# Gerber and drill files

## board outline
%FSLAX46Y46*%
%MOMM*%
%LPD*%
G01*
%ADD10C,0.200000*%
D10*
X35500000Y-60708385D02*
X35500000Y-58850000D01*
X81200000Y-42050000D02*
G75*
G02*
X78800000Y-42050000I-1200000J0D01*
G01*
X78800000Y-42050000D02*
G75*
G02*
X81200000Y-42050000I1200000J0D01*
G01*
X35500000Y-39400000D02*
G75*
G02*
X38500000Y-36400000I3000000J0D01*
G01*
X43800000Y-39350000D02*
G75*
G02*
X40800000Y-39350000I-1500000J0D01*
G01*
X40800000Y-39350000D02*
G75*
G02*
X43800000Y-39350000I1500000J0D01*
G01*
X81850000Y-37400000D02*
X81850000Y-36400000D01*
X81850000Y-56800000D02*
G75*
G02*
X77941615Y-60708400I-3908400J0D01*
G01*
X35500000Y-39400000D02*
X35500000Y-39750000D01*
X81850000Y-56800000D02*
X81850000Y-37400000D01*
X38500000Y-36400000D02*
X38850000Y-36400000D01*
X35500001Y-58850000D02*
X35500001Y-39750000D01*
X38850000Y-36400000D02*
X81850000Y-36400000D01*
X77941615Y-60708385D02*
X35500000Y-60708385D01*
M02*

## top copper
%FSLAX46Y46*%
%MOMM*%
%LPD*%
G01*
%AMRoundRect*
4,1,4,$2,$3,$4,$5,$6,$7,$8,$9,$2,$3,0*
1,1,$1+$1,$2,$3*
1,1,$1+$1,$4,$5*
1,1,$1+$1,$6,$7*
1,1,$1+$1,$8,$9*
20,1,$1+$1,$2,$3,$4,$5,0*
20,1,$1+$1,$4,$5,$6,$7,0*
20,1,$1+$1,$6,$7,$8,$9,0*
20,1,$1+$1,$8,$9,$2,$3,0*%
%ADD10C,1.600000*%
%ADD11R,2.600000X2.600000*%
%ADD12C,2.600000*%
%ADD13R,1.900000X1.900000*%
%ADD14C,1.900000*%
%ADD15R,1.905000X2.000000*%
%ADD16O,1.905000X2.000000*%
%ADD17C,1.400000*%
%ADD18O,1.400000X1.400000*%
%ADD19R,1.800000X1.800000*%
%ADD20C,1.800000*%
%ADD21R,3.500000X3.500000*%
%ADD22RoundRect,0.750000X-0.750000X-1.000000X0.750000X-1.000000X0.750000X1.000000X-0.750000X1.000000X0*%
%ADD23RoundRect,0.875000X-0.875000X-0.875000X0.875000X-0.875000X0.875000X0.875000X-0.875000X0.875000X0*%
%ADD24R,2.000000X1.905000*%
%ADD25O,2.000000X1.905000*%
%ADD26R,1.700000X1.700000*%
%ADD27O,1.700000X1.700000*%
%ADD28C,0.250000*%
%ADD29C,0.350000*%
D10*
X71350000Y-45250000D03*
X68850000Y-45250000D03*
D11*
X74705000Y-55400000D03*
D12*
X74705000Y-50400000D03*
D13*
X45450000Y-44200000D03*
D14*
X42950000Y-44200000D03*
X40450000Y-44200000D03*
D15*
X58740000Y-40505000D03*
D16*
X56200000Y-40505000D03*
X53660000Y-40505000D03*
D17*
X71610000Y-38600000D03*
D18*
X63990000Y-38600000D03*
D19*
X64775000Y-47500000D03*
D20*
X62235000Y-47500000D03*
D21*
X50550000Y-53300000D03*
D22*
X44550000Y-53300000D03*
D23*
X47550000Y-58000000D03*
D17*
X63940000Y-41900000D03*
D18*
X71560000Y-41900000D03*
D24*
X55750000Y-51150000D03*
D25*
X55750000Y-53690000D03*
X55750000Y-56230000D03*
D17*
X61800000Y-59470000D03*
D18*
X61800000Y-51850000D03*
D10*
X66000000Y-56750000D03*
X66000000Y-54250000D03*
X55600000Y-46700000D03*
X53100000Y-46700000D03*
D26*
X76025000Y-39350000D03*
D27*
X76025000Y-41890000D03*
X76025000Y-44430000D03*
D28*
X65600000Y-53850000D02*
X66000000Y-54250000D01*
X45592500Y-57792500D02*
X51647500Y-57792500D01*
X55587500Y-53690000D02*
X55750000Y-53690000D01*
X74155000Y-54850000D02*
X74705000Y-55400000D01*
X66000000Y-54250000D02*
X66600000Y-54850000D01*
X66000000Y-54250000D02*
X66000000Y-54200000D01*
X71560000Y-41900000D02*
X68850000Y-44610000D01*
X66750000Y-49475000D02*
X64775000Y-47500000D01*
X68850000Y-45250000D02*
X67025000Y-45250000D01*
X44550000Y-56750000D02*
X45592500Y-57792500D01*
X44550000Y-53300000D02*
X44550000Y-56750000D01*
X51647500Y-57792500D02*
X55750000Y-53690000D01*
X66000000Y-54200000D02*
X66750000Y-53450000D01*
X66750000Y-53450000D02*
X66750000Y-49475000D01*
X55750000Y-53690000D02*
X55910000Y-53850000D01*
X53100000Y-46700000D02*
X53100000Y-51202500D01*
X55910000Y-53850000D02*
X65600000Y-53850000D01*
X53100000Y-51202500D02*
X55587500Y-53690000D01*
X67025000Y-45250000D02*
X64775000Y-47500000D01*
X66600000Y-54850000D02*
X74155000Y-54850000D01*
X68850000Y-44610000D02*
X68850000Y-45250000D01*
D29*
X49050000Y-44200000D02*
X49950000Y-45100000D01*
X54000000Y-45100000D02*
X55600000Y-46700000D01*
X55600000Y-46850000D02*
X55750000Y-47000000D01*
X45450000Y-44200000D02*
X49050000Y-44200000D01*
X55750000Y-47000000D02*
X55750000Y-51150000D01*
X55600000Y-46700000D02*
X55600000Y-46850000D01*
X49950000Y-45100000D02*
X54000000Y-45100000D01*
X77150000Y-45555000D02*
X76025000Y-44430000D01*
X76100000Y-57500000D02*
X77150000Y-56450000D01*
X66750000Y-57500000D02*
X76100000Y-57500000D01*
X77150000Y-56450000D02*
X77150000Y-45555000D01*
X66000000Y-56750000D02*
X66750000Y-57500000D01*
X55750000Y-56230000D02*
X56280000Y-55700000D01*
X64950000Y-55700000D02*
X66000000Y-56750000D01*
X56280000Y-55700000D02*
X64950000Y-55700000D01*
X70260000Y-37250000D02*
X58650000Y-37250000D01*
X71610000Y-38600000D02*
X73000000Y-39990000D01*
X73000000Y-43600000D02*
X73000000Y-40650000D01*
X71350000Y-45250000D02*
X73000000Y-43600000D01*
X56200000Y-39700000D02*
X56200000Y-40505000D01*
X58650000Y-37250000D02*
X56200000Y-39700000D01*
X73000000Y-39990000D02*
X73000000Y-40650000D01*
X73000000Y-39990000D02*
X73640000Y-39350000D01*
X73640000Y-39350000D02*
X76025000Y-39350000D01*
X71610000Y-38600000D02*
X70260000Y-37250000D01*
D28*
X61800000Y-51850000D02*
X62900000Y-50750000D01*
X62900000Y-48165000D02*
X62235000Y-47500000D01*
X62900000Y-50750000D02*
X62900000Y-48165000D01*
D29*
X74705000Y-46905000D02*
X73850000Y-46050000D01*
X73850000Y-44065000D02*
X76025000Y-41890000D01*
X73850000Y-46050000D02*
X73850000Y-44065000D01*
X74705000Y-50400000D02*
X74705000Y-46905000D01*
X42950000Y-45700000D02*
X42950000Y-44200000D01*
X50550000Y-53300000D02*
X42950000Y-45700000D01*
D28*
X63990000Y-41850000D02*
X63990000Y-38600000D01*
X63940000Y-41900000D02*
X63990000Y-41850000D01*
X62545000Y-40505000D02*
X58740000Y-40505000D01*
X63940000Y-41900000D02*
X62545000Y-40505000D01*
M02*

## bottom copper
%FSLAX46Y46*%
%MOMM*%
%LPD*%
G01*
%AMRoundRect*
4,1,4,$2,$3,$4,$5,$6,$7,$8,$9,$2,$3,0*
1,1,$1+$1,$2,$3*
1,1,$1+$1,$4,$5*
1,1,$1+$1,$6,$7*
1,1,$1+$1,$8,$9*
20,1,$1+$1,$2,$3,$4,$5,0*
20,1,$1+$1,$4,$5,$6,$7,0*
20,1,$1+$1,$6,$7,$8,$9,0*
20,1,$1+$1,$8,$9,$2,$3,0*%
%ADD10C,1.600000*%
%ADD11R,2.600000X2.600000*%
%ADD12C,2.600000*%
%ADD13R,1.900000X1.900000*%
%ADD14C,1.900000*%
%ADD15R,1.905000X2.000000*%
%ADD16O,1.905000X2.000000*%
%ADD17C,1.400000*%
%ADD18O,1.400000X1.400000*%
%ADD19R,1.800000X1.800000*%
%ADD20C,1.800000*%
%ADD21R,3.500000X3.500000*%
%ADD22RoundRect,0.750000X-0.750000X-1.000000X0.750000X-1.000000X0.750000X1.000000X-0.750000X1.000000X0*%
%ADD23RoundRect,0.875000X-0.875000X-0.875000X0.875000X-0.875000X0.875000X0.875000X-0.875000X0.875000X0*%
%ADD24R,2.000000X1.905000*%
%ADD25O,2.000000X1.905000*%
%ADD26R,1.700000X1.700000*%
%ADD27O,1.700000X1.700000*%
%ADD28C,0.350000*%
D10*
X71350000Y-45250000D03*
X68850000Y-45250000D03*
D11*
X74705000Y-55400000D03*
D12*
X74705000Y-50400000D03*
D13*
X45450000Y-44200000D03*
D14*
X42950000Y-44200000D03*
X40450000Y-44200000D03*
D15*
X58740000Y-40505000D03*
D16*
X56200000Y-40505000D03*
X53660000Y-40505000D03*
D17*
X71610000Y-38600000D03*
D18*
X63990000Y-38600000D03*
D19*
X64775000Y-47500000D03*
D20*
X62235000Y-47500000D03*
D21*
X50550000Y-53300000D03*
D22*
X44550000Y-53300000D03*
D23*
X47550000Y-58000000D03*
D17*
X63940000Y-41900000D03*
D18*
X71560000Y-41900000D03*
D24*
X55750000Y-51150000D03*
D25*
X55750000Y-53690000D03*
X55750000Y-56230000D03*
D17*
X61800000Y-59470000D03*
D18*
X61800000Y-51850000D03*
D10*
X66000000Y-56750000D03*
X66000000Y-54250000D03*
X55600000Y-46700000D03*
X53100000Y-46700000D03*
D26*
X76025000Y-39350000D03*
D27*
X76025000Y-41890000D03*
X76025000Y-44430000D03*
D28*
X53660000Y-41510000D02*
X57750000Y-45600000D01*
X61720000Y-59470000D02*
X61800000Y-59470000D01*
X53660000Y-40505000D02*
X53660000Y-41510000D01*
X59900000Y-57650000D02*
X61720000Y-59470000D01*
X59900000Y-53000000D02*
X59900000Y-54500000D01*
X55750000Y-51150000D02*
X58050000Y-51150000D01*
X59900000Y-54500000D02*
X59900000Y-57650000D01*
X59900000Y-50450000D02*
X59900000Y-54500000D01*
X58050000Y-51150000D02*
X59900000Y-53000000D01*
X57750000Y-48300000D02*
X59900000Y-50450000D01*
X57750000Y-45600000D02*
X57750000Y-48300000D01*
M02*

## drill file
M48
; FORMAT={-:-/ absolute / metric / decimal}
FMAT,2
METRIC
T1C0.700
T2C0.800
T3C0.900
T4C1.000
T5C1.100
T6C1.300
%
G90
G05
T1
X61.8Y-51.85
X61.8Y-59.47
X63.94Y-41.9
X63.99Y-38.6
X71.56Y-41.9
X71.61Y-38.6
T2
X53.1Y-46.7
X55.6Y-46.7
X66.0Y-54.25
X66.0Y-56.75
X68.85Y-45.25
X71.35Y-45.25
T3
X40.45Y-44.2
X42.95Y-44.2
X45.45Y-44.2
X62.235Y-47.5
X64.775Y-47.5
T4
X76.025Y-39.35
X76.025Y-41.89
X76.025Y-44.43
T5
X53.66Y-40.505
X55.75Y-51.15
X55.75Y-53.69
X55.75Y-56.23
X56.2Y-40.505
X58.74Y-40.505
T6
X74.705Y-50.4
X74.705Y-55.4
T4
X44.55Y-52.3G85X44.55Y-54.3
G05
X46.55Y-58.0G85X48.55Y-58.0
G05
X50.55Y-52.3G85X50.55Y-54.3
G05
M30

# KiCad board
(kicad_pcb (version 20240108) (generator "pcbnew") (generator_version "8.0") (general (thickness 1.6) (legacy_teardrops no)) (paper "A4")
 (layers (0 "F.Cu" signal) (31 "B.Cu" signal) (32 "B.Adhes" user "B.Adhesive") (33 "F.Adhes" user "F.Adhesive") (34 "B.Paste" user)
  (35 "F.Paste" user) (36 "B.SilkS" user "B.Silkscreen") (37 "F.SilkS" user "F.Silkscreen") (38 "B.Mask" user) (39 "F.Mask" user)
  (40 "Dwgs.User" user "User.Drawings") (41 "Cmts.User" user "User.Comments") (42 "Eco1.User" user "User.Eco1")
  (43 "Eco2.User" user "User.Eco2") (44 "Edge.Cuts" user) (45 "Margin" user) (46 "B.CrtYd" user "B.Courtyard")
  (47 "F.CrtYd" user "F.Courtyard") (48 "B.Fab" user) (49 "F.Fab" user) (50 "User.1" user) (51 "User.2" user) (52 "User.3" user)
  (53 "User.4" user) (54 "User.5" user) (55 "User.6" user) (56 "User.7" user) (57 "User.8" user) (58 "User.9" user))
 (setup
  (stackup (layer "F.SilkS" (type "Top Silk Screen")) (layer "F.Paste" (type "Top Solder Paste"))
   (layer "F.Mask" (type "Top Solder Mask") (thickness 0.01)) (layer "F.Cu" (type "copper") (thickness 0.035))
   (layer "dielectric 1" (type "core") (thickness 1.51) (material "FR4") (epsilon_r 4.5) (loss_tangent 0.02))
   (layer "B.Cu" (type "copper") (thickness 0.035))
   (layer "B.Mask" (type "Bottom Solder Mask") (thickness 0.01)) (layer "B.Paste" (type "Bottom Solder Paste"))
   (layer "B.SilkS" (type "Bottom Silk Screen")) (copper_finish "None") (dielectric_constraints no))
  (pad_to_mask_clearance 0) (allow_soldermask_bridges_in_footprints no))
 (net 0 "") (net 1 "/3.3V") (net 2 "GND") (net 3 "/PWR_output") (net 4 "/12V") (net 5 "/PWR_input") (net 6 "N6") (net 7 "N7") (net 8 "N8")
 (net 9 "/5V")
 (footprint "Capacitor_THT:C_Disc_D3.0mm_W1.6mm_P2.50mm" (layer "F.Cu") (at 71.35 45.25 180)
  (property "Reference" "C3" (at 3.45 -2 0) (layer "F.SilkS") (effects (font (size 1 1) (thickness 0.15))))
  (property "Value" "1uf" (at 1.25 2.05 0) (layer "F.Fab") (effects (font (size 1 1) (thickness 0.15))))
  (pad "1" thru_hole circle (at 0 0 180) (size 1.6 1.6) (drill 0.8) (layers "*.Cu" "*.Mask") (remove_unused_layers no) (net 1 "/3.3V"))
  (pad "2" thru_hole circle (at 2.5 0 180) (size 1.6 1.6) (drill 0.8) (layers "*.Cu" "*.Mask") (remove_unused_layers no) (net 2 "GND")))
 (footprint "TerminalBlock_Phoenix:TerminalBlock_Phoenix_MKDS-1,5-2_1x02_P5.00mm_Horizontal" (layer "F.Cu") (at 74.705 55.4 90)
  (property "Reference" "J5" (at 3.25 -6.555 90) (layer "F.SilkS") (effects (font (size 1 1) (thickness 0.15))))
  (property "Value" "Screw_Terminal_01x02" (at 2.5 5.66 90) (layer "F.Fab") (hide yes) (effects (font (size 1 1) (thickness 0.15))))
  (pad "1" thru_hole rect (at 0 0 90) (size 2.6 2.6) (drill 1.3) (layers "*.Cu" "*.Mask") (remove_unused_layers no) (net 2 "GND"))
  (pad "2" thru_hole circle (at 5 0 90) (size 2.6 2.6) (drill 1.3) (layers "*.Cu" "*.Mask") (remove_unused_layers no) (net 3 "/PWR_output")))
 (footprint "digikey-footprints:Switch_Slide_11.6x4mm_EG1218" (layer "F.Cu") (at 45.45 44.2 180)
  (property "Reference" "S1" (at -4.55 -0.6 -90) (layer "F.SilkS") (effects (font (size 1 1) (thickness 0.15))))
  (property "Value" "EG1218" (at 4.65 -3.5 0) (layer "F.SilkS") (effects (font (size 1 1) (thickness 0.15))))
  (pad "1" thru_hole rect (at 0 0 180) (size 1.9 1.9) (drill 0.9) (layers "*.Cu" "*.Mask") (remove_unused_layers no) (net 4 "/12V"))
  (pad "2" thru_hole circle (at 2.5 0 180) (size 1.9 1.9) (drill 0.9) (layers "*.Cu" "*.Mask") (remove_unused_layers no)
   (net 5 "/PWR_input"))
  (pad "3" thru_hole circle (at 5 0 180) (size 1.9 1.9) (drill 0.9) (layers "*.Cu" "*.Mask") (remove_unused_layers no) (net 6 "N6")))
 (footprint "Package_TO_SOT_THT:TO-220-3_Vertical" (layer "F.Cu") (at 58.74 40.505 180)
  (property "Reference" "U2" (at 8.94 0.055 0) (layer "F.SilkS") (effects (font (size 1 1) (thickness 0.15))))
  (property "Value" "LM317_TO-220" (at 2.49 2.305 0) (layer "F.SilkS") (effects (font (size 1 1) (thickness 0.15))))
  (pad "1" thru_hole rect (at 0 0 180) (size 1.905 2) (drill 1.1) (layers "*.Cu" "*.Mask") (remove_unused_layers no) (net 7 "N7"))
  (pad "2" thru_hole oval (at 2.54 0 180) (size 1.905 2) (drill 1.1) (layers "*.Cu" "*.Mask") (remove_unused_layers no) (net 1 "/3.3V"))
  (pad "3" thru_hole oval (at 5.08 0 180) (size 1.905 2) (drill 1.1) (layers "*.Cu" "*.Mask") (remove_unused_layers no) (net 4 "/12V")))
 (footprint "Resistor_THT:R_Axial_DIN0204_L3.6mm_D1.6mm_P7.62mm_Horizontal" (layer "F.Cu") (at 71.61 38.6 180)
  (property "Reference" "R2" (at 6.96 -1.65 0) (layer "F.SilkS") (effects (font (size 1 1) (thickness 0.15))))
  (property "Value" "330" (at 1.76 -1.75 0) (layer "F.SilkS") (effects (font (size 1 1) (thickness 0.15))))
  (pad "1" thru_hole circle (at 0 0 180) (size 1.4 1.4) (drill 0.7) (layers "*.Cu" "*.Mask") (remove_unused_layers no) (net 1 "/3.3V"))
  (pad "2" thru_hole oval (at 7.62 0 180) (size 1.4 1.4) (drill 0.7) (layers "*.Cu" "*.Mask") (remove_unused_layers no) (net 7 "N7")))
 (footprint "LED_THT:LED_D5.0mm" (layer "F.Cu") (at 64.775 47.5 180)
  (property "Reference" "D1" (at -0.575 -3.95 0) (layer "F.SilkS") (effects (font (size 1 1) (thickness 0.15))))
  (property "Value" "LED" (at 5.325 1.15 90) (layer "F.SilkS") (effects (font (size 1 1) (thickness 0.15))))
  (pad "1" thru_hole rect (at 0 0 180) (size 1.8 1.8) (drill 0.9) (layers "*.Cu" "*.Mask") (remove_unused_layers no) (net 2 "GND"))
  (pad "2" thru_hole circle (at 2.54 0 180) (size 1.8 1.8) (drill 0.9) (layers "*.Cu" "*.Mask") (remove_unused_layers no) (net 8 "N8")))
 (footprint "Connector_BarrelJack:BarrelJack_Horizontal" (layer "F.Cu") (at 50.55 53.3)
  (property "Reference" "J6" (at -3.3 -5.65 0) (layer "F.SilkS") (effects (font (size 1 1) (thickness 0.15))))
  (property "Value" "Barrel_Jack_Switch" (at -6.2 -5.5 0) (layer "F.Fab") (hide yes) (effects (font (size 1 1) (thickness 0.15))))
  (pad "1" thru_hole rect (at 0 0) (size 3.5 3.5) (drill oval 1 3) (layers "*.Cu" "*.Mask") (remove_unused_layers no) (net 5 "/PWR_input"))
  (pad "2" thru_hole roundrect (at -6 0) (size 3 3.5) (drill oval 1 3) (layers "*.Cu" "*.Mask") (remove_unused_layers no)
   (roundrect_rratio 0.25) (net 2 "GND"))
  (pad "3" thru_hole roundrect (at -3 4.7) (size 3.5 3.5) (drill oval 3 1) (layers "*.Cu" "*.Mask") (remove_unused_layers no)
   (roundrect_rratio 0.25) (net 2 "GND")))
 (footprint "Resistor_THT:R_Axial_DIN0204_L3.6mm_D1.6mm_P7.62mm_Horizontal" (layer "F.Cu") (at 63.94 41.9)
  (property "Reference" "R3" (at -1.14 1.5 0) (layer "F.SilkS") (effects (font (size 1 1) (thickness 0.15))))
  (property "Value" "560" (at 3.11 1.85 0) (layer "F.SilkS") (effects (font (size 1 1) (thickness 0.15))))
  (pad "1" thru_hole circle (at 0 0) (size 1.4 1.4) (drill 0.7) (layers "*.Cu" "*.Mask") (remove_unused_layers no) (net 7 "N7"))
  (pad "2" thru_hole oval (at 7.62 0) (size 1.4 1.4) (drill 0.7) (layers "*.Cu" "*.Mask") (remove_unused_layers no) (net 2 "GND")))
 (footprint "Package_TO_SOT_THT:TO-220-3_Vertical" (layer "F.Cu") (at 55.75 51.15 -90)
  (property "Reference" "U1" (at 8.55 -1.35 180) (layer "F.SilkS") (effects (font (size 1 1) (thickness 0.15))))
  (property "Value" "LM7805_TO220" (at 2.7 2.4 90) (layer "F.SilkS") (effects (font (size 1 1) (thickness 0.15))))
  (pad "1" thru_hole rect (at 0 0 270) (size 1.905 2) (drill 1.1) (layers "*.Cu" "*.Mask") (remove_unused_layers no) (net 4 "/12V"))
  (pad "2" thru_hole oval (at 2.54 0 270) (size 1.905 2) (drill 1.1) (layers "*.Cu" "*.Mask") (remove_unused_layers no) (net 2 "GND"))
  (pad "3" thru_hole oval (at 5.08 0 270) (size 1.905 2) (drill 1.1) (layers "*.Cu" "*.Mask") (remove_unused_layers no) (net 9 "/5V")))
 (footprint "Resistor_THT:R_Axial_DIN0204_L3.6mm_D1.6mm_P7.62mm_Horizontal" (layer "F.Cu") (at 61.8 59.47 90)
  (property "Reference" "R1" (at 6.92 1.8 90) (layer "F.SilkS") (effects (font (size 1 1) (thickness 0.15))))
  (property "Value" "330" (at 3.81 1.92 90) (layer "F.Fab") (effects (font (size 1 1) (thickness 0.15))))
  (pad "1" thru_hole circle (at 0 0 90) (size 1.4 1.4) (drill 0.7) (layers "*.Cu" "*.Mask") (remove_unused_layers no) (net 4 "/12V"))
  (pad "2" thru_hole oval (at 7.62 0 90) (size 1.4 1.4) (drill 0.7) (layers "*.Cu" "*.Mask") (remove_unused_layers no) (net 8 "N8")))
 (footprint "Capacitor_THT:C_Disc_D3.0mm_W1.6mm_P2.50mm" (layer "F.Cu") (at 66 56.75 90)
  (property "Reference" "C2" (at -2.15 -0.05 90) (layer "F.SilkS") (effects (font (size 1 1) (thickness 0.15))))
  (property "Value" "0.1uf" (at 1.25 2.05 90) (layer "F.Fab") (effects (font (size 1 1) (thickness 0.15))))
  (pad "1" thru_hole circle (at 0 0 90) (size 1.6 1.6) (drill 0.8) (layers "*.Cu" "*.Mask") (remove_unused_layers no) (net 9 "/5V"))
  (pad "2" thru_hole circle (at 2.5 0 90) (size 1.6 1.6) (drill 0.8) (layers "*.Cu" "*.Mask") (remove_unused_layers no) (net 2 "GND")))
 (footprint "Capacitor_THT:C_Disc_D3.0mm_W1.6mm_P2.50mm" (layer "F.Cu") (at 55.6 46.7 180)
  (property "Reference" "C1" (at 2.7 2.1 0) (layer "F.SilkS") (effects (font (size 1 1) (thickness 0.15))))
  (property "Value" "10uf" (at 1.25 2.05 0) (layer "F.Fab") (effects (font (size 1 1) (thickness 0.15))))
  (pad "1" thru_hole circle (at 0 0 180) (size 1.6 1.6) (drill 0.8) (layers "*.Cu" "*.Mask") (remove_unused_layers no) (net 4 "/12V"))
  (pad "2" thru_hole circle (at 2.5 0 180) (size 1.6 1.6) (drill 0.8) (layers "*.Cu" "*.Mask") (remove_unused_layers no) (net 2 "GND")))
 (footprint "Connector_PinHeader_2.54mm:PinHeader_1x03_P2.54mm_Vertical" (layer "F.Cu") (at 76.025 39.35)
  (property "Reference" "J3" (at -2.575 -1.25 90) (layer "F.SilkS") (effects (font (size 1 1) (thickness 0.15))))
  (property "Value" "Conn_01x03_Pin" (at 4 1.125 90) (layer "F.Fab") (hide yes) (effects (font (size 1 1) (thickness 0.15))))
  (pad "1" thru_hole rect (at 0 0) (size 1.7 1.7) (drill 1) (layers "*.Cu" "*.Mask") (remove_unused_layers no) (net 1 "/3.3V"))
  (pad "2" thru_hole oval (at 0 2.54) (size 1.7 1.7) (drill 1) (layers "*.Cu" "*.Mask") (remove_unused_layers no) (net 3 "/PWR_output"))
  (pad "3" thru_hole oval (at 0 5.08) (size 1.7 1.7) (drill 1) (layers "*.Cu" "*.Mask") (remove_unused_layers no) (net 9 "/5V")))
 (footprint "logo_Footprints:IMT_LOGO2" (layer "F.Cu") (at 43.000889 40.072258)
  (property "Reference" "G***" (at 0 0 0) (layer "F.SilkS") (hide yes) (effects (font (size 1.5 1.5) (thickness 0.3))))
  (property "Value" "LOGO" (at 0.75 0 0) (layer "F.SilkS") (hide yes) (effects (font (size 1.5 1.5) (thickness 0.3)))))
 (gr_line (start 35.5 60.708385) (end 35.5 58.85) (stroke (width 0.2) (type default)) (layer "Edge.Cuts"))
 (gr_circle (center 80 42.05) (end 81.2 42.05) (stroke (width 0.2) (type default)) (fill none) (layer "Edge.Cuts"))
 (gr_arc (start 35.5 39.4) (mid 36.37868 37.27868) (end 38.5 36.4) (stroke (width 0.2) (type default)) (layer "Edge.Cuts"))
 (gr_circle (center 42.3 39.35) (end 43.8 39.35) (stroke (width 0.2) (type default)) (fill none) (layer "Edge.Cuts"))
 (gr_line (start 81.85 37.4) (end 81.85 36.4) (stroke (width 0.2) (type default)) (layer "Edge.Cuts"))
 (gr_arc (start 81.85 56.8) (mid 80.705261 59.563646) (end 77.941615 60.708385) (stroke (width 0.2) (type default)) (layer "Edge.Cuts"))
 (gr_line (start 35.5 39.4) (end 35.5 39.75) (stroke (width 0.2) (type default)) (layer "Edge.Cuts"))
 (gr_line (start 81.85 56.8) (end 81.85 37.4) (stroke (width 0.2) (type default)) (layer "Edge.Cuts"))
 (gr_line (start 38.5 36.4) (end 38.85 36.4) (stroke (width 0.2) (type default)) (layer "Edge.Cuts"))
 (gr_line (start 35.500001 58.85) (end 35.500001 39.75) (stroke (width 0.2) (type default)) (layer "Edge.Cuts"))
 (gr_line (start 38.85 36.4) (end 81.85 36.4) (stroke (width 0.2) (type default)) (layer "Edge.Cuts"))
 (gr_line (start 77.941615 60.708385) (end 35.5 60.708385) (stroke (width 0.2) (type default)) (layer "Edge.Cuts"))
 (segment (start 65.6 53.85) (end 66 54.25) (width 0.25) (layer "F.Cu") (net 2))
 (segment (start 45.5925 57.7925) (end 51.6475 57.7925) (width 0.25) (layer "F.Cu") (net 2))
 (segment (start 55.5875 53.69) (end 55.75 53.69) (width 0.25) (layer "F.Cu") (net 2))
 (segment (start 74.155 54.85) (end 74.705 55.4) (width 0.25) (layer "F.Cu") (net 2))
 (segment (start 66 54.25) (end 66.6 54.85) (width 0.25) (layer "F.Cu") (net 2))
 (segment (start 66 54.25) (end 66 54.2) (width 0.25) (layer "F.Cu") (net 2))
 (segment (start 71.56 41.9) (end 68.85 44.61) (width 0.25) (layer "F.Cu") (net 2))
 (segment (start 66.75 49.475) (end 64.775 47.5) (width 0.25) (layer "F.Cu") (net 2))
 (segment (start 68.85 45.25) (end 67.025 45.25) (width 0.25) (layer "F.Cu") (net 2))
 (segment (start 44.55 56.75) (end 45.5925 57.7925) (width 0.25) (layer "F.Cu") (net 2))
 (segment (start 44.55 53.3) (end 44.55 56.75) (width 0.25) (layer "F.Cu") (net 2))
 (segment (start 51.6475 57.7925) (end 55.75 53.69) (width 0.25) (layer "F.Cu") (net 2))
 (segment (start 66 54.2) (end 66.75 53.45) (width 0.25) (layer "F.Cu") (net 2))
 (segment (start 66.75 53.45) (end 66.75 49.475) (width 0.25) (layer "F.Cu") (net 2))
 (segment (start 55.75 53.69) (end 55.91 53.85) (width 0.25) (layer "F.Cu") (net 2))
 (segment (start 53.1 46.7) (end 53.1 51.2025) (width 0.25) (layer "F.Cu") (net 2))
 (segment (start 55.91 53.85) (end 65.6 53.85) (width 0.25) (layer "F.Cu") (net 2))
 (segment (start 53.1 51.2025) (end 55.5875 53.69) (width 0.25) (layer "F.Cu") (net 2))
 (segment (start 67.025 45.25) (end 64.775 47.5) (width 0.25) (layer "F.Cu") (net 2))
 (segment (start 66.6 54.85) (end 74.155 54.85) (width 0.25) (layer "F.Cu") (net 2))
 (segment (start 68.85 44.61) (end 68.85 45.25) (width 0.25) (layer "F.Cu") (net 2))
 (segment (start 49.05 44.2) (end 49.95 45.1) (width 0.35) (layer "F.Cu") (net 4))
 (segment (start 54 45.1) (end 55.6 46.7) (width 0.35) (layer "F.Cu") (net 4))
 (segment (start 55.6 46.85) (end 55.75 47) (width 0.35) (layer "F.Cu") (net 4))
 (segment (start 45.45 44.2) (end 49.05 44.2) (width 0.35) (layer "F.Cu") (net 4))
 (segment (start 55.75 47) (end 55.75 51.15) (width 0.35) (layer "F.Cu") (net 4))
 (segment (start 55.6 46.7) (end 55.6 46.85) (width 0.35) (layer "F.Cu") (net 4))
 (segment (start 49.95 45.1) (end 54 45.1) (width 0.35) (layer "F.Cu") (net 4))
 (segment (start 53.66 41.51) (end 57.75 45.6) (width 0.35) (layer "B.Cu") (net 4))
 (segment (start 61.72 59.47) (end 61.8 59.47) (width 0.35) (layer "B.Cu") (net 4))
 (segment (start 53.66 40.505) (end 53.66 41.51) (width 0.35) (layer "B.Cu") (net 4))
 (segment (start 59.9 57.65) (end 61.72 59.47) (width 0.35) (layer "B.Cu") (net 4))
 (segment (start 59.9 53) (end 59.9 54.5) (width 0.35) (layer "B.Cu") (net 4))
 (segment (start 55.75 51.15) (end 58.05 51.15) (width 0.35) (layer "B.Cu") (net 4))
 (segment (start 59.9 54.5) (end 59.9 57.65) (width 0.35) (layer "B.Cu") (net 4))
 (segment (start 59.9 50.45) (end 59.9 54.5) (width 0.35) (layer "B.Cu") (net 4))
 (segment (start 58.05 51.15) (end 59.9 53) (width 0.35) (layer "B.Cu") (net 4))
 (segment (start 57.75 48.3) (end 59.9 50.45) (width 0.35) (layer "B.Cu") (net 4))
 (segment (start 57.75 45.6) (end 57.75 48.3) (width 0.35) (layer "B.Cu") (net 4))
 (segment (start 77.15 45.555) (end 76.025 44.43) (width 0.35) (layer "F.Cu") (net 9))
 (segment (start 76.1 57.5) (end 77.15 56.45) (width 0.35) (layer "F.Cu") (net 9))
 (segment (start 66.75 57.5) (end 76.1 57.5) (width 0.35) (layer "F.Cu") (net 9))
 (segment (start 77.15 56.45) (end 77.15 45.555) (width 0.35) (layer "F.Cu") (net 9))
 (segment (start 66 56.75) (end 66.75 57.5) (width 0.35) (layer "F.Cu") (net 9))
 (segment (start 55.75 56.23) (end 56.28 55.7) (width 0.35) (layer "F.Cu") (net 9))
 (segment (start 64.95 55.7) (end 66 56.75) (width 0.35) (layer "F.Cu") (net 9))
 (segment (start 56.28 55.7) (end 64.95 55.7) (width 0.35) (layer "F.Cu") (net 9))
 (segment (start 70.26 37.25) (end 58.65 37.25) (width 0.35) (layer "F.Cu") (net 1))
 (segment (start 71.61 38.6) (end 73 39.99) (width 0.35) (layer "F.Cu") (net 1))
 (segment (start 73 43.6) (end 73 40.65) (width 0.35) (layer "F.Cu") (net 1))
 (segment (start 71.35 45.25) (end 73 43.6) (width 0.35) (layer "F.Cu") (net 1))
 (segment (start 56.2 39.7) (end 56.2 40.505) (width 0.35) (layer "F.Cu") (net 1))
 (segment (start 58.65 37.25) (end 56.2 39.7) (width 0.35) (layer "F.Cu") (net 1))
 (segment (start 73 39.99) (end 73 40.65) (width 0.35) (layer "F.Cu") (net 1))
 (segment (start 73 39.99) (end 73.64 39.35) (width 0.35) (layer "F.Cu") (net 1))
 (segment (start 73.64 39.35) (end 76.025 39.35) (width 0.35) (layer "F.Cu") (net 1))
 (segment (start 71.61 38.6) (end 70.26 37.25) (width 0.35) (layer "F.Cu") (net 1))
 (segment (start 61.8 51.85) (end 62.9 50.75) (width 0.25) (layer "F.Cu") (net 8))
 (segment (start 62.9 48.165) (end 62.235 47.5) (width 0.25) (layer "F.Cu") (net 8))
 (segment (start 62.9 50.75) (end 62.9 48.165) (width 0.25) (layer "F.Cu") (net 8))
 (segment (start 74.705 46.905) (end 73.85 46.05) (width 0.35) (layer "F.Cu") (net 3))
 (segment (start 73.85 44.065) (end 76.025 41.89) (width 0.35) (layer "F.Cu") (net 3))
 (segment (start 73.85 46.05) (end 73.85 44.065) (width 0.35) (layer "F.Cu") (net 3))
 (segment (start 74.705 50.4) (end 74.705 46.905) (width 0.35) (layer "F.Cu") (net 3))
 (segment (start 42.95 45.7) (end 42.95 44.2) (width 0.35) (layer "F.Cu") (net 5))
 (segment (start 50.55 53.3) (end 42.95 45.7) (width 0.35) (layer "F.Cu") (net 5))
 (segment (start 63.99 41.85) (end 63.99 38.6) (width 0.25) (layer "F.Cu") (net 7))
 (segment (start 63.94 41.9) (end 63.99 41.85) (width 0.25) (layer "F.Cu") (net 7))
 (segment (start 62.545 40.505) (end 58.74 40.505) (width 0.25) (layer "F.Cu") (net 7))
 (segment (start 63.94 41.9) (end 62.545 40.505) (width 0.25) (layer "F.Cu") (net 7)))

